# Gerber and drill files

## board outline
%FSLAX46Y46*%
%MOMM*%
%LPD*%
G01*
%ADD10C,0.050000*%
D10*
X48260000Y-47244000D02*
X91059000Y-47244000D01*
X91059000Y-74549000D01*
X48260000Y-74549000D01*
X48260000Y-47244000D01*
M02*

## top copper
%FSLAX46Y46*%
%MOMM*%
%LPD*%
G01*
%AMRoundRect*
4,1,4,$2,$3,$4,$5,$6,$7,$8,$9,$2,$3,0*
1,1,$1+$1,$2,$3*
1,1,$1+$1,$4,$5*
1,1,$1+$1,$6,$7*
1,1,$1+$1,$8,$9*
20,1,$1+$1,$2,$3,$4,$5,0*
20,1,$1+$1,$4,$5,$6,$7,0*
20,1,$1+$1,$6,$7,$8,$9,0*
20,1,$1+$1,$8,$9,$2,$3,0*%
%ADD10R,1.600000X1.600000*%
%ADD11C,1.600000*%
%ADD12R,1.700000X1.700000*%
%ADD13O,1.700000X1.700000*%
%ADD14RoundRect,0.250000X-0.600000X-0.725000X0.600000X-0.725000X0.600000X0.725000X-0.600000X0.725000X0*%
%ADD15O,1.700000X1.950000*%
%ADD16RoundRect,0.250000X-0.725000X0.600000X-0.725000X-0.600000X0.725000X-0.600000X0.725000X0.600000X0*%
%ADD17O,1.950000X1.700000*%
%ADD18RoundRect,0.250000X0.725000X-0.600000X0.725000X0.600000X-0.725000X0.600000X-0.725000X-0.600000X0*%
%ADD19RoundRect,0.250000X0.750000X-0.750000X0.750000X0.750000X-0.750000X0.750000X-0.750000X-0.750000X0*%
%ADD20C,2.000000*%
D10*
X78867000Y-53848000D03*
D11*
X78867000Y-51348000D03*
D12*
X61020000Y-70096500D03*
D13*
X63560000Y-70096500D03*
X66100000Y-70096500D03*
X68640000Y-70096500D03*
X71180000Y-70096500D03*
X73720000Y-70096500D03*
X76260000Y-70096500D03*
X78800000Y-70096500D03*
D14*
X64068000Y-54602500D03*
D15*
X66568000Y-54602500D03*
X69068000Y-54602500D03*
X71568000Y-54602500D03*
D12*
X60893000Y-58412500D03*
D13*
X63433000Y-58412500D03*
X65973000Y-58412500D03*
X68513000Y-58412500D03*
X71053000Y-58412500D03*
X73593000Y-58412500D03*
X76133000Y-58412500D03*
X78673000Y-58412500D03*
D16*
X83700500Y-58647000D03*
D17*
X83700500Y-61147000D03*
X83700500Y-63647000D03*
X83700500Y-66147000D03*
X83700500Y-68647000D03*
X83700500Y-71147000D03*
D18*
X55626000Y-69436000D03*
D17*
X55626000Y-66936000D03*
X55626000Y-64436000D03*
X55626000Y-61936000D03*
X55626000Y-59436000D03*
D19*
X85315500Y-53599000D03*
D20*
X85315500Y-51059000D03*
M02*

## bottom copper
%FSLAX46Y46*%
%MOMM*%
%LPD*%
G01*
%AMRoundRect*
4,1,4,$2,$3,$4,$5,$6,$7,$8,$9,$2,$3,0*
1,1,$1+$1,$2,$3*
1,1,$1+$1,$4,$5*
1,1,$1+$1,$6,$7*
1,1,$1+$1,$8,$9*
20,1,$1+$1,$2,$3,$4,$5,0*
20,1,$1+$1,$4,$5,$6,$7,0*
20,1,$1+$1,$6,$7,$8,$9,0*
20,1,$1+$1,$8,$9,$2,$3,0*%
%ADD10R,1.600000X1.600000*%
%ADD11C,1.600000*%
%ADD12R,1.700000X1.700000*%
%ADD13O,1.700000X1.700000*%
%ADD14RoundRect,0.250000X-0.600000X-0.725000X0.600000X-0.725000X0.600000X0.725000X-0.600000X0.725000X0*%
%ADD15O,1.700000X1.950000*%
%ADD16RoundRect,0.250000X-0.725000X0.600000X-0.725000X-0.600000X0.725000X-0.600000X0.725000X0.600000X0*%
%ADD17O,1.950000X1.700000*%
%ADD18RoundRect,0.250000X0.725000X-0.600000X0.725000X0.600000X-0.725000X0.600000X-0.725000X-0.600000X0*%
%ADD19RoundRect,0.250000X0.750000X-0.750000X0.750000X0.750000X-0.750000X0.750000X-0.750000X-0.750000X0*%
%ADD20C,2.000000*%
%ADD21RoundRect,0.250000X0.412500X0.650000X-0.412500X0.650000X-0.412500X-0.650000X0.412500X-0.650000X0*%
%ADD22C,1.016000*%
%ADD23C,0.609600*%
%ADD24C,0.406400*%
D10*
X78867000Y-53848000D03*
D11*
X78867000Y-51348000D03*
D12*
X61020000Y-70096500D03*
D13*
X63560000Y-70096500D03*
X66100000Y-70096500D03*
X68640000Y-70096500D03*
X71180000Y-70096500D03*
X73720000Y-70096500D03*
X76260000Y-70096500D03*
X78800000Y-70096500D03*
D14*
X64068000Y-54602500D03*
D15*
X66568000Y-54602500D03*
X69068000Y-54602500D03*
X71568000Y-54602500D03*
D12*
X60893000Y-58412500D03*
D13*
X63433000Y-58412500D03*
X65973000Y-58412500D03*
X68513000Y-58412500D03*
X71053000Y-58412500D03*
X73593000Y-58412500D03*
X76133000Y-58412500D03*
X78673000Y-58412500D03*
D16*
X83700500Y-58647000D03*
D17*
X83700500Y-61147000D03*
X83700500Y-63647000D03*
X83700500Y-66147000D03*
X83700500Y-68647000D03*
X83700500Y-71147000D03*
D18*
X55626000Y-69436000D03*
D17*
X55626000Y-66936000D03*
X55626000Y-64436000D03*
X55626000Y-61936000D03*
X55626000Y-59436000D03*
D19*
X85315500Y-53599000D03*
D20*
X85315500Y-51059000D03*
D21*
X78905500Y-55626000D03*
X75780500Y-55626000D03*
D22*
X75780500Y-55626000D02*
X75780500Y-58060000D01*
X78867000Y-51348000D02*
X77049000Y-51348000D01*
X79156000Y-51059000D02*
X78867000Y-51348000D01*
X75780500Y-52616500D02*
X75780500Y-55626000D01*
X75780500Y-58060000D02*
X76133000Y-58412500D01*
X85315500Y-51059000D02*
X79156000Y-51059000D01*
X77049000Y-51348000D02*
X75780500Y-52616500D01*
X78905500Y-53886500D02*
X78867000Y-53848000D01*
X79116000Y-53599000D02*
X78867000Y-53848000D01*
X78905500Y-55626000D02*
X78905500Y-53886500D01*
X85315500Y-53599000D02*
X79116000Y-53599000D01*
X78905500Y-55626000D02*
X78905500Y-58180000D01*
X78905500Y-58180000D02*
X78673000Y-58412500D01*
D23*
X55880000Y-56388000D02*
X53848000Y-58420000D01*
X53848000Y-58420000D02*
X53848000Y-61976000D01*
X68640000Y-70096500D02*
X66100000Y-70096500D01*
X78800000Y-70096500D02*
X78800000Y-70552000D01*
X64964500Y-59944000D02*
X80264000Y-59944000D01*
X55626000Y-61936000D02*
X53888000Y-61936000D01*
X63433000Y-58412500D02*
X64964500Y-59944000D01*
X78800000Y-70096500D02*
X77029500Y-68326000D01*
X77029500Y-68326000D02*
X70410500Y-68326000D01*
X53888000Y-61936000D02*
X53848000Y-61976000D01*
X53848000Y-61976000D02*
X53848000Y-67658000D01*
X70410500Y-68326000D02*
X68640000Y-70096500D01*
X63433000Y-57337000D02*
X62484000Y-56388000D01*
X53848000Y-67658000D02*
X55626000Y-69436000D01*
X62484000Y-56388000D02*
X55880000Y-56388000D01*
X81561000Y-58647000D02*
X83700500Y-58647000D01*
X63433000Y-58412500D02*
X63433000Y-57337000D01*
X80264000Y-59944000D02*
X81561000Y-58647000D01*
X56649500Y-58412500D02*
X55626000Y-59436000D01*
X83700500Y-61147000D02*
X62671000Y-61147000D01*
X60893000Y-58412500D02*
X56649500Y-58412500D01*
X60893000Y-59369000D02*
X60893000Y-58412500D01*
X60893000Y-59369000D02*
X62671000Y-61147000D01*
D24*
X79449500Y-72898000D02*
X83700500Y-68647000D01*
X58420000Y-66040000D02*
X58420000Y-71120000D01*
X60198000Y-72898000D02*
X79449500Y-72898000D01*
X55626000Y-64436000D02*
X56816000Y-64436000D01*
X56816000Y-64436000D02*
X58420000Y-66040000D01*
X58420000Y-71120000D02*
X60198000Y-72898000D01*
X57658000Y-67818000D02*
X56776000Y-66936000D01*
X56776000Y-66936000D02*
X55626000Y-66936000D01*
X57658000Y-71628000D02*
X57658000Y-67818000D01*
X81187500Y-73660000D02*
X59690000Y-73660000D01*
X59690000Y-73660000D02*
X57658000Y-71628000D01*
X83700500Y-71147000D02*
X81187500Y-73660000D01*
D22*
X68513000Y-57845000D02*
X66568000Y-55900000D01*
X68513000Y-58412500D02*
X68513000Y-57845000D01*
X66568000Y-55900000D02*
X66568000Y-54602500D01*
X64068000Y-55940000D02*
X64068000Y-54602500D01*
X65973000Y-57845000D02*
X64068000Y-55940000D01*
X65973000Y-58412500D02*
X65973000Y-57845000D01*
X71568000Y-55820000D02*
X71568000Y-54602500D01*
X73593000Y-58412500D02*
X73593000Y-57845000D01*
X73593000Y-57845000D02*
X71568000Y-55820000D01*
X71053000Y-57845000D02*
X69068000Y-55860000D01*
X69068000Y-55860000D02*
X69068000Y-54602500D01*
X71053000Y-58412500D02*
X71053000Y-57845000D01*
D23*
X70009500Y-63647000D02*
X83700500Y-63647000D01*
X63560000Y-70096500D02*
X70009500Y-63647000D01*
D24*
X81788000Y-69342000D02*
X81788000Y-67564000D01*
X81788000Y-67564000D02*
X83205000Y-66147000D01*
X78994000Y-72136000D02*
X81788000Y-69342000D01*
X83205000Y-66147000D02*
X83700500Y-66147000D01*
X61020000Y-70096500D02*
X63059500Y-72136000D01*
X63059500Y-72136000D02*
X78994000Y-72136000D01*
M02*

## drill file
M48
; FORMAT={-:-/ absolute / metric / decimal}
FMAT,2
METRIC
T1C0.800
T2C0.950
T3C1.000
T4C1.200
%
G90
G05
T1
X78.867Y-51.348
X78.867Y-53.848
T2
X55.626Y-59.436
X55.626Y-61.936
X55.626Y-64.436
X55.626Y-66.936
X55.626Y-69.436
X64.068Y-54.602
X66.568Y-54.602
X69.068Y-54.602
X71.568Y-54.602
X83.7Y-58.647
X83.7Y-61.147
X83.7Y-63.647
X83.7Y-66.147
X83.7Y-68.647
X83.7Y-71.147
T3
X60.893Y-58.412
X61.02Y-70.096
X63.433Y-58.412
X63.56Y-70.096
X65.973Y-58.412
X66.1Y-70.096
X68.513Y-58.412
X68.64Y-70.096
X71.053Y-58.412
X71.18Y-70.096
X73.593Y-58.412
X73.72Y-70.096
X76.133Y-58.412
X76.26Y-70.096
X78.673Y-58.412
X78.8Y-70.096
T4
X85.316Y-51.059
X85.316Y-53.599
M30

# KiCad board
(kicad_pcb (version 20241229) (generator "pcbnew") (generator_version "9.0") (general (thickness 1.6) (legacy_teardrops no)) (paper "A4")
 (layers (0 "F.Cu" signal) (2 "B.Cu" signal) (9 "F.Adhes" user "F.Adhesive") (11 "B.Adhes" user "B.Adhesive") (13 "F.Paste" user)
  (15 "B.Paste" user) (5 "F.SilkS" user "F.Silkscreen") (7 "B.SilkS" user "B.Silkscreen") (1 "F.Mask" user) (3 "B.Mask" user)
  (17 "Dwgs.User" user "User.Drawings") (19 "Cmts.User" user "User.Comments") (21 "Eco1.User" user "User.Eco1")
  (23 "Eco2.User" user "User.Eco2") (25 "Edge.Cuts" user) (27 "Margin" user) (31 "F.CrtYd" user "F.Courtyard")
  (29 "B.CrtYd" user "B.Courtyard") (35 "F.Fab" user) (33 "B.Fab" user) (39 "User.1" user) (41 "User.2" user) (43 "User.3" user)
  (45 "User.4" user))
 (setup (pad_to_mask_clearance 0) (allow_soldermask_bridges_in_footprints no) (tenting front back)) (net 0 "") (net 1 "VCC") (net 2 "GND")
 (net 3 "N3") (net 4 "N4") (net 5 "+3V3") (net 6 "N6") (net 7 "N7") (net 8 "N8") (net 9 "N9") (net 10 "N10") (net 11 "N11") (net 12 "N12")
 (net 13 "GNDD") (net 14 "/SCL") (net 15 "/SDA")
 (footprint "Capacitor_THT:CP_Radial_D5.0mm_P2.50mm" (layer "F.Cu") (at 78.867 53.848 90)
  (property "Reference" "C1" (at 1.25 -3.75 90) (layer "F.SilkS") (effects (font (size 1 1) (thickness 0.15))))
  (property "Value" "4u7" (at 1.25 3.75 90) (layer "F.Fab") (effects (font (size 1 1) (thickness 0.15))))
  (pad "1" thru_hole rect (at 0 0 90) (size 1.6 1.6) (drill 0.8) (layers "*.Cu" "*.Mask") (remove_unused_layers no) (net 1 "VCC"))
  (pad "2" thru_hole circle (at 2.5 0 90) (size 1.6 1.6) (drill 0.8) (layers "*.Cu" "*.Mask") (remove_unused_layers no) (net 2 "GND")))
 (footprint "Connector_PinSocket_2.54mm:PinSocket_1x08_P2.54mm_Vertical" (layer "F.Cu") (at 61.02 70.0965 90)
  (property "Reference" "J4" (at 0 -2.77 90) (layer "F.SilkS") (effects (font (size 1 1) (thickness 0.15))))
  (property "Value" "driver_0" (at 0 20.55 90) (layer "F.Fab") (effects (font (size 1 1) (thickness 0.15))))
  (pad "1" thru_hole rect (at 0 0 90) (size 1.7 1.7) (drill 1) (layers "*.Cu" "*.Mask") (remove_unused_layers no) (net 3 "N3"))
  (pad "2" thru_hole oval (at 0 2.54 90) (size 1.7 1.7) (drill 1) (layers "*.Cu" "*.Mask") (remove_unused_layers no) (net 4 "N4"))
  (pad "3" thru_hole oval (at 0 5.08 90) (size 1.7 1.7) (drill 1) (layers "*.Cu" "*.Mask") (remove_unused_layers no) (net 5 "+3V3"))
  (pad "4" thru_hole oval (at 0 7.62 90) (size 1.7 1.7) (drill 1) (layers "*.Cu" "*.Mask") (remove_unused_layers no) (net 5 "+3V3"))
  (pad "5" thru_hole oval (at 0 10.16 90) (size 1.7 1.7) (drill 1) (layers "*.Cu" "*.Mask") (remove_unused_layers no) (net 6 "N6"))
  (pad "6" thru_hole oval (at 0 12.7 90) (size 1.7 1.7) (drill 1) (layers "*.Cu" "*.Mask") (remove_unused_layers no) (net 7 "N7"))
  (pad "7" thru_hole oval (at 0 15.24 90) (size 1.7 1.7) (drill 1) (layers "*.Cu" "*.Mask") (remove_unused_layers no) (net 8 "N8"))
  (pad "8" thru_hole oval (at 0 17.78 90) (size 1.7 1.7) (drill 1) (layers "*.Cu" "*.Mask") (remove_unused_layers no) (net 5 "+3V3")))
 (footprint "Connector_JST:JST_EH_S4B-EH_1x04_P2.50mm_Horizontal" (layer "F.Cu") (at 64.068 54.6025)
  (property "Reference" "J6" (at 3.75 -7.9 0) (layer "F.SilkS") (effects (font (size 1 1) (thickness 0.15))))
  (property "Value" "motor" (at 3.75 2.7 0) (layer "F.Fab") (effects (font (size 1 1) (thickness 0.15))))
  (pad "1" thru_hole roundrect (at 0 0) (size 1.7 1.95) (drill 0.95) (layers "*.Cu" "*.Mask") (remove_unused_layers no)
   (roundrect_rratio 0.147059) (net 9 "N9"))
  (pad "2" thru_hole oval (at 2.5 0) (size 1.7 1.95) (drill 0.95) (layers "*.Cu" "*.Mask") (remove_unused_layers no) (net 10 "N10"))
  (pad "3" thru_hole oval (at 5 0) (size 1.7 1.95) (drill 0.95) (layers "*.Cu" "*.Mask") (remove_unused_layers no) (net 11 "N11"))
  (pad "4" thru_hole oval (at 7.5 0) (size 1.7 1.95) (drill 0.95) (layers "*.Cu" "*.Mask") (remove_unused_layers no) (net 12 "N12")))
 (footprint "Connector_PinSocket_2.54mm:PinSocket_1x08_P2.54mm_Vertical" (layer "F.Cu") (at 60.893 58.4125 90)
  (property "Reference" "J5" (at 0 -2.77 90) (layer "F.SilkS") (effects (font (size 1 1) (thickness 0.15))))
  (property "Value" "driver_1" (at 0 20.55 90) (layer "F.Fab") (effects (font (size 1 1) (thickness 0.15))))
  (pad "1" thru_hole rect (at 0 0 90) (size 1.7 1.7) (drill 1) (layers "*.Cu" "*.Mask") (remove_unused_layers no) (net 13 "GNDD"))
  (pad "2" thru_hole oval (at 0 2.54 90) (size 1.7 1.7) (drill 1) (layers "*.Cu" "*.Mask") (remove_unused_layers no) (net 5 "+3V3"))
  (pad "3" thru_hole oval (at 0 5.08 90) (size 1.7 1.7) (drill 1) (layers "*.Cu" "*.Mask") (remove_unused_layers no) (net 9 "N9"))
  (pad "4" thru_hole oval (at 0 7.62 90) (size 1.7 1.7) (drill 1) (layers "*.Cu" "*.Mask") (remove_unused_layers no) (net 10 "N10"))
  (pad "5" thru_hole oval (at 0 10.16 90) (size 1.7 1.7) (drill 1) (layers "*.Cu" "*.Mask") (remove_unused_layers no) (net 11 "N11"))
  (pad "6" thru_hole oval (at 0 12.7 90) (size 1.7 1.7) (drill 1) (layers "*.Cu" "*.Mask") (remove_unused_layers no) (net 12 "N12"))
  (pad "7" thru_hole oval (at 0 15.24 90) (size 1.7 1.7) (drill 1) (layers "*.Cu" "*.Mask") (remove_unused_layers no) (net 2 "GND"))
  (pad "8" thru_hole oval (at 0 17.78 90) (size 1.7 1.7) (drill 1) (layers "*.Cu" "*.Mask") (remove_unused_layers no) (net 1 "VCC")))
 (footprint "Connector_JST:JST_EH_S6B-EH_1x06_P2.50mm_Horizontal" (layer "F.Cu") (at 83.7005 58.647 -90)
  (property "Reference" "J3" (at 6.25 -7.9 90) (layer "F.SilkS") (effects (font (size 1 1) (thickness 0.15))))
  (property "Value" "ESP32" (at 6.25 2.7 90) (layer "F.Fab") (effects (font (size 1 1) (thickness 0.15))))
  (pad "1" thru_hole roundrect (at 0 0 270) (size 1.7 1.95) (drill 0.95) (layers "*.Cu" "*.Mask") (remove_unused_layers no)
   (roundrect_rratio 0.147059) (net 5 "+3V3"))
  (pad "2" thru_hole oval (at 2.5 0 270) (size 1.7 1.95) (drill 0.95) (layers "*.Cu" "*.Mask") (remove_unused_layers no) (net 13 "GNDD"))
  (pad "3" thru_hole oval (at 5 0 270) (size 1.7 1.95) (drill 0.95) (layers "*.Cu" "*.Mask") (remove_unused_layers no) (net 4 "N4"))
  (pad "4" thru_hole oval (at 7.5 0 270) (size 1.7 1.95) (drill 0.95) (layers "*.Cu" "*.Mask") (remove_unused_layers no) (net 3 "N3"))
  (pad "5" thru_hole oval (at 10 0 270) (size 1.7 1.95) (drill 0.95) (layers "*.Cu" "*.Mask") (remove_unused_layers no) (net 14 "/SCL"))
  (pad "6" thru_hole oval (at 12.5 0 270) (size 1.7 1.95) (drill 0.95) (layers "*.Cu" "*.Mask") (remove_unused_layers no) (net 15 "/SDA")))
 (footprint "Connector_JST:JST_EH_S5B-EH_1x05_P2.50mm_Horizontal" (layer "F.Cu") (at 55.626 69.436 90)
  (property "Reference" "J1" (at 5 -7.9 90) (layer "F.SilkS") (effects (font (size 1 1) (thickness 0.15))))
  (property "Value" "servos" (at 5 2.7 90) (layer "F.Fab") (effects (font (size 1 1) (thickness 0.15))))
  (pad "1" thru_hole roundrect (at 0 0 90) (size 1.7 1.95) (drill 0.95) (layers "*.Cu" "*.Mask") (remove_unused_layers no)
   (roundrect_rratio 0.147059) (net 5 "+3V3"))
  (pad "2" thru_hole oval (at 2.5 0 90) (size 1.7 1.95) (drill 0.95) (layers "*.Cu" "*.Mask") (remove_unused_layers no) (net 15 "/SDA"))
  (pad "3" thru_hole oval (at 5 0 90) (size 1.7 1.95) (drill 0.95) (layers "*.Cu" "*.Mask") (remove_unused_layers no) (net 14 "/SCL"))
  (pad "4" thru_hole oval (at 7.5 0 90) (size 1.7 1.95) (drill 0.95) (layers "*.Cu" "*.Mask") (remove_unused_layers no) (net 5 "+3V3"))
  (pad "5" thru_hole oval (at 10 0 90) (size 1.7 1.95) (drill 0.95) (layers "*.Cu" "*.Mask") (remove_unused_layers no) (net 13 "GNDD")))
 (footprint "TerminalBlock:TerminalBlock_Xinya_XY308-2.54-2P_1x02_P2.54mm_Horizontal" (layer "F.Cu") (at 85.3155 53.599 90)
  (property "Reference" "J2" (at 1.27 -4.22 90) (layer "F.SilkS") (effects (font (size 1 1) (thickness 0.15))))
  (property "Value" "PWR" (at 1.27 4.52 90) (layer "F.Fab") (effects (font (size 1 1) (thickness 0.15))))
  (pad "1" thru_hole roundrect (at 0 0 90) (size 2 2) (drill 1.2) (layers "*.Cu" "*.Mask") (remove_unused_layers no)
   (roundrect_rratio 0.125) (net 1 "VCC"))
  (pad "2" thru_hole circle (at 2.54 0 90) (size 2 2) (drill 1.2) (layers "*.Cu" "*.Mask") (remove_unused_layers no) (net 2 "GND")))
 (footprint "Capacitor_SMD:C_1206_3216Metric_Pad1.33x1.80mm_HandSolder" (layer "B.Cu") (at 77.343 55.626 180)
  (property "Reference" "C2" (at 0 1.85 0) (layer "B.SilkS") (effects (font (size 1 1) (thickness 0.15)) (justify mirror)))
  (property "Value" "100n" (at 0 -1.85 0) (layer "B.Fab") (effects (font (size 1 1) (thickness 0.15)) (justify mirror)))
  (pad "1" smd roundrect (at -1.5625 0 180) (size 1.325 1.8) (layers "B.Cu" "B.Mask" "B.Paste") (roundrect_rratio 0.188679) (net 1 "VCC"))
  (pad "2" smd roundrect (at 1.5625 0 180) (size 1.325 1.8) (layers "B.Cu" "B.Mask" "B.Paste") (roundrect_rratio 0.188679) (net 2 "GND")))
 (gr_rect (start 48.26 47.244) (end 91.059 74.549) (stroke (width 0.05) (type default)) (fill no) (layer "Edge.Cuts"))
 (segment (start 75.7805 55.626) (end 75.7805 58.06) (width 1.016) (layer "B.Cu") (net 2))
 (segment (start 78.867 51.348) (end 77.049 51.348) (width 1.016) (layer "B.Cu") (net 2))
 (segment (start 79.156 51.059) (end 78.867 51.348) (width 1.016) (layer "B.Cu") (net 2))
 (segment (start 75.7805 52.6165) (end 75.7805 55.626) (width 1.016) (layer "B.Cu") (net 2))
 (segment (start 75.7805 58.06) (end 76.133 58.4125) (width 1.016) (layer "B.Cu") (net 2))
 (segment (start 85.3155 51.059) (end 79.156 51.059) (width 1.016) (layer "B.Cu") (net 2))
 (segment (start 77.049 51.348) (end 75.7805 52.6165) (width 1.016) (layer "B.Cu") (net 2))
 (segment (start 78.9055 53.8865) (end 78.867 53.848) (width 1.016) (layer "B.Cu") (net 1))
 (segment (start 79.116 53.599) (end 78.867 53.848) (width 1.016) (layer "B.Cu") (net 1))
 (segment (start 78.9055 55.626) (end 78.9055 53.8865) (width 1.016) (layer "B.Cu") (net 1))
 (segment (start 85.3155 53.599) (end 79.116 53.599) (width 1.016) (layer "B.Cu") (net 1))
 (segment (start 78.9055 55.626) (end 78.9055 58.18) (width 1.016) (layer "B.Cu") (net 1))
 (segment (start 78.9055 58.18) (end 78.673 58.4125) (width 1.016) (layer "B.Cu") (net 1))
 (segment (start 55.88 56.388) (end 53.848 58.42) (width 0.6096) (layer "B.Cu") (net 5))
 (segment (start 53.848 58.42) (end 53.848 61.976) (width 0.6096) (layer "B.Cu") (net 5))
 (segment (start 68.64 70.0965) (end 66.1 70.0965) (width 0.6096) (layer "B.Cu") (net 5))
 (segment (start 78.8 70.0965) (end 78.8 70.552) (width 0.6096) (layer "B.Cu") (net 5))
 (segment (start 64.9645 59.944) (end 80.264 59.944) (width 0.6096) (layer "B.Cu") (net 5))
 (segment (start 55.626 61.936) (end 53.888 61.936) (width 0.6096) (layer "B.Cu") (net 5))
 (segment (start 63.433 58.4125) (end 64.9645 59.944) (width 0.6096) (layer "B.Cu") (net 5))
 (segment (start 78.8 70.0965) (end 77.0295 68.326) (width 0.6096) (layer "B.Cu") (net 5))
 (segment (start 77.0295 68.326) (end 70.4105 68.326) (width 0.6096) (layer "B.Cu") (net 5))
 (segment (start 53.888 61.936) (end 53.848 61.976) (width 0.6096) (layer "B.Cu") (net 5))
 (segment (start 53.848 61.976) (end 53.848 67.658) (width 0.6096) (layer "B.Cu") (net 5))
 (segment (start 70.4105 68.326) (end 68.64 70.0965) (width 0.6096) (layer "B.Cu") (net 5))
 (segment (start 63.433 57.337) (end 62.484 56.388) (width 0.6096) (layer "B.Cu") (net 5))
 (segment (start 53.848 67.658) (end 55.626 69.436) (width 0.6096) (layer "B.Cu") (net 5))
 (segment (start 62.484 56.388) (end 55.88 56.388) (width 0.6096) (layer "B.Cu") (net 5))
 (segment (start 81.561 58.647) (end 83.7005 58.647) (width 0.6096) (layer "B.Cu") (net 5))
 (segment (start 63.433 58.4125) (end 63.433 57.337) (width 0.6096) (layer "B.Cu") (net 5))
 (segment (start 80.264 59.944) (end 81.561 58.647) (width 0.6096) (layer "B.Cu") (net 5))
 (segment (start 56.6495 58.4125) (end 55.626 59.436) (width 0.6096) (layer "B.Cu") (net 13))
 (segment (start 83.7005 61.147) (end 62.671 61.147) (width 0.6096) (layer "B.Cu") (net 13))
 (segment (start 60.893 58.4125) (end 56.6495 58.4125) (width 0.6096) (layer "B.Cu") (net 13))
 (segment (start 60.893 59.369) (end 60.893 58.4125) (width 0.6096) (layer "B.Cu") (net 13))
 (segment (start 60.893 59.369) (end 62.671 61.147) (width 0.6096) (layer "B.Cu") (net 13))
 (segment (start 79.4495 72.898) (end 83.7005 68.647) (width 0.4064) (layer "B.Cu") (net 14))
 (segment (start 58.42 66.04) (end 58.42 71.12) (width 0.4064) (layer "B.Cu") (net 14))
 (segment (start 60.198 72.898) (end 79.4495 72.898) (width 0.4064) (layer "B.Cu") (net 14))
 (segment (start 55.626 64.436) (end 56.816 64.436) (width 0.4064) (layer "B.Cu") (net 14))
 (segment (start 56.816 64.436) (end 58.42 66.04) (width 0.4064) (layer "B.Cu") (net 14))
 (segment (start 58.42 71.12) (end 60.198 72.898) (width 0.4064) (layer "B.Cu") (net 14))
 (segment (start 57.658 67.818) (end 56.776 66.936) (width 0.4064) (layer "B.Cu") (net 15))
 (segment (start 56.776 66.936) (end 55.626 66.936) (width 0.4064) (layer "B.Cu") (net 15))
 (segment (start 57.658 71.628) (end 57.658 67.818) (width 0.4064) (layer "B.Cu") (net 15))
 (segment (start 81.1875 73.66) (end 59.69 73.66) (width 0.4064) (layer "B.Cu") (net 15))
 (segment (start 59.69 73.66) (end 57.658 71.628) (width 0.4064) (layer "B.Cu") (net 15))
 (segment (start 83.7005 71.147) (end 81.1875 73.66) (width 0.4064) (layer "B.Cu") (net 15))
 (segment (start 68.513 57.845) (end 66.568 55.9) (width 1.016) (layer "B.Cu") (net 10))
 (segment (start 68.513 58.4125) (end 68.513 57.845) (width 1.016) (layer "B.Cu") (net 10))
 (segment (start 66.568 55.9) (end 66.568 54.6025) (width 1.016) (layer "B.Cu") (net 10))
 (segment (start 64.068 55.94) (end 64.068 54.6025) (width 1.016) (layer "B.Cu") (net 9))
 (segment (start 65.973 57.845) (end 64.068 55.94) (width 1.016) (layer "B.Cu") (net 9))
 (segment (start 65.973 58.4125) (end 65.973 57.845) (width 1.016) (layer "B.Cu") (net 9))
 (segment (start 71.568 55.82) (end 71.568 54.6025) (width 1.016) (layer "B.Cu") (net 12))
 (segment (start 73.593 58.4125) (end 73.593 57.845) (width 1.016) (layer "B.Cu") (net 12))
 (segment (start 73.593 57.845) (end 71.568 55.82) (width 1.016) (layer "B.Cu") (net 12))
 (segment (start 71.053 57.845) (end 69.068 55.86) (width 1.016) (layer "B.Cu") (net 11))
 (segment (start 69.068 55.86) (end 69.068 54.6025) (width 1.016) (layer "B.Cu") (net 11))
 (segment (start 71.053 58.4125) (end 71.053 57.845) (width 1.016) (layer "B.Cu") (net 11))
 (segment (start 70.0095 63.647) (end 83.7005 63.647) (width 0.6096) (layer "B.Cu") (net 4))
 (segment (start 63.56 70.0965) (end 70.0095 63.647) (width 0.6096) (layer "B.Cu") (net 4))
 (segment (start 81.788 69.342) (end 81.788 67.564) (width 0.4064) (layer "B.Cu") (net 3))
 (segment (start 81.788 67.564) (end 83.205 66.147) (width 0.4064) (layer "B.Cu") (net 3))
 (segment (start 78.994 72.136) (end 81.788 69.342) (width 0.4064) (layer "B.Cu") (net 3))
 (segment (start 83.205 66.147) (end 83.7005 66.147) (width 0.4064) (layer "B.Cu") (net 3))
 (segment (start 61.02 70.0965) (end 63.0595 72.136) (width 0.4064) (layer "B.Cu") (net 3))
 (segment (start 63.0595 72.136) (end 78.994 72.136) (width 0.4064) (layer "B.Cu") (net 3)))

